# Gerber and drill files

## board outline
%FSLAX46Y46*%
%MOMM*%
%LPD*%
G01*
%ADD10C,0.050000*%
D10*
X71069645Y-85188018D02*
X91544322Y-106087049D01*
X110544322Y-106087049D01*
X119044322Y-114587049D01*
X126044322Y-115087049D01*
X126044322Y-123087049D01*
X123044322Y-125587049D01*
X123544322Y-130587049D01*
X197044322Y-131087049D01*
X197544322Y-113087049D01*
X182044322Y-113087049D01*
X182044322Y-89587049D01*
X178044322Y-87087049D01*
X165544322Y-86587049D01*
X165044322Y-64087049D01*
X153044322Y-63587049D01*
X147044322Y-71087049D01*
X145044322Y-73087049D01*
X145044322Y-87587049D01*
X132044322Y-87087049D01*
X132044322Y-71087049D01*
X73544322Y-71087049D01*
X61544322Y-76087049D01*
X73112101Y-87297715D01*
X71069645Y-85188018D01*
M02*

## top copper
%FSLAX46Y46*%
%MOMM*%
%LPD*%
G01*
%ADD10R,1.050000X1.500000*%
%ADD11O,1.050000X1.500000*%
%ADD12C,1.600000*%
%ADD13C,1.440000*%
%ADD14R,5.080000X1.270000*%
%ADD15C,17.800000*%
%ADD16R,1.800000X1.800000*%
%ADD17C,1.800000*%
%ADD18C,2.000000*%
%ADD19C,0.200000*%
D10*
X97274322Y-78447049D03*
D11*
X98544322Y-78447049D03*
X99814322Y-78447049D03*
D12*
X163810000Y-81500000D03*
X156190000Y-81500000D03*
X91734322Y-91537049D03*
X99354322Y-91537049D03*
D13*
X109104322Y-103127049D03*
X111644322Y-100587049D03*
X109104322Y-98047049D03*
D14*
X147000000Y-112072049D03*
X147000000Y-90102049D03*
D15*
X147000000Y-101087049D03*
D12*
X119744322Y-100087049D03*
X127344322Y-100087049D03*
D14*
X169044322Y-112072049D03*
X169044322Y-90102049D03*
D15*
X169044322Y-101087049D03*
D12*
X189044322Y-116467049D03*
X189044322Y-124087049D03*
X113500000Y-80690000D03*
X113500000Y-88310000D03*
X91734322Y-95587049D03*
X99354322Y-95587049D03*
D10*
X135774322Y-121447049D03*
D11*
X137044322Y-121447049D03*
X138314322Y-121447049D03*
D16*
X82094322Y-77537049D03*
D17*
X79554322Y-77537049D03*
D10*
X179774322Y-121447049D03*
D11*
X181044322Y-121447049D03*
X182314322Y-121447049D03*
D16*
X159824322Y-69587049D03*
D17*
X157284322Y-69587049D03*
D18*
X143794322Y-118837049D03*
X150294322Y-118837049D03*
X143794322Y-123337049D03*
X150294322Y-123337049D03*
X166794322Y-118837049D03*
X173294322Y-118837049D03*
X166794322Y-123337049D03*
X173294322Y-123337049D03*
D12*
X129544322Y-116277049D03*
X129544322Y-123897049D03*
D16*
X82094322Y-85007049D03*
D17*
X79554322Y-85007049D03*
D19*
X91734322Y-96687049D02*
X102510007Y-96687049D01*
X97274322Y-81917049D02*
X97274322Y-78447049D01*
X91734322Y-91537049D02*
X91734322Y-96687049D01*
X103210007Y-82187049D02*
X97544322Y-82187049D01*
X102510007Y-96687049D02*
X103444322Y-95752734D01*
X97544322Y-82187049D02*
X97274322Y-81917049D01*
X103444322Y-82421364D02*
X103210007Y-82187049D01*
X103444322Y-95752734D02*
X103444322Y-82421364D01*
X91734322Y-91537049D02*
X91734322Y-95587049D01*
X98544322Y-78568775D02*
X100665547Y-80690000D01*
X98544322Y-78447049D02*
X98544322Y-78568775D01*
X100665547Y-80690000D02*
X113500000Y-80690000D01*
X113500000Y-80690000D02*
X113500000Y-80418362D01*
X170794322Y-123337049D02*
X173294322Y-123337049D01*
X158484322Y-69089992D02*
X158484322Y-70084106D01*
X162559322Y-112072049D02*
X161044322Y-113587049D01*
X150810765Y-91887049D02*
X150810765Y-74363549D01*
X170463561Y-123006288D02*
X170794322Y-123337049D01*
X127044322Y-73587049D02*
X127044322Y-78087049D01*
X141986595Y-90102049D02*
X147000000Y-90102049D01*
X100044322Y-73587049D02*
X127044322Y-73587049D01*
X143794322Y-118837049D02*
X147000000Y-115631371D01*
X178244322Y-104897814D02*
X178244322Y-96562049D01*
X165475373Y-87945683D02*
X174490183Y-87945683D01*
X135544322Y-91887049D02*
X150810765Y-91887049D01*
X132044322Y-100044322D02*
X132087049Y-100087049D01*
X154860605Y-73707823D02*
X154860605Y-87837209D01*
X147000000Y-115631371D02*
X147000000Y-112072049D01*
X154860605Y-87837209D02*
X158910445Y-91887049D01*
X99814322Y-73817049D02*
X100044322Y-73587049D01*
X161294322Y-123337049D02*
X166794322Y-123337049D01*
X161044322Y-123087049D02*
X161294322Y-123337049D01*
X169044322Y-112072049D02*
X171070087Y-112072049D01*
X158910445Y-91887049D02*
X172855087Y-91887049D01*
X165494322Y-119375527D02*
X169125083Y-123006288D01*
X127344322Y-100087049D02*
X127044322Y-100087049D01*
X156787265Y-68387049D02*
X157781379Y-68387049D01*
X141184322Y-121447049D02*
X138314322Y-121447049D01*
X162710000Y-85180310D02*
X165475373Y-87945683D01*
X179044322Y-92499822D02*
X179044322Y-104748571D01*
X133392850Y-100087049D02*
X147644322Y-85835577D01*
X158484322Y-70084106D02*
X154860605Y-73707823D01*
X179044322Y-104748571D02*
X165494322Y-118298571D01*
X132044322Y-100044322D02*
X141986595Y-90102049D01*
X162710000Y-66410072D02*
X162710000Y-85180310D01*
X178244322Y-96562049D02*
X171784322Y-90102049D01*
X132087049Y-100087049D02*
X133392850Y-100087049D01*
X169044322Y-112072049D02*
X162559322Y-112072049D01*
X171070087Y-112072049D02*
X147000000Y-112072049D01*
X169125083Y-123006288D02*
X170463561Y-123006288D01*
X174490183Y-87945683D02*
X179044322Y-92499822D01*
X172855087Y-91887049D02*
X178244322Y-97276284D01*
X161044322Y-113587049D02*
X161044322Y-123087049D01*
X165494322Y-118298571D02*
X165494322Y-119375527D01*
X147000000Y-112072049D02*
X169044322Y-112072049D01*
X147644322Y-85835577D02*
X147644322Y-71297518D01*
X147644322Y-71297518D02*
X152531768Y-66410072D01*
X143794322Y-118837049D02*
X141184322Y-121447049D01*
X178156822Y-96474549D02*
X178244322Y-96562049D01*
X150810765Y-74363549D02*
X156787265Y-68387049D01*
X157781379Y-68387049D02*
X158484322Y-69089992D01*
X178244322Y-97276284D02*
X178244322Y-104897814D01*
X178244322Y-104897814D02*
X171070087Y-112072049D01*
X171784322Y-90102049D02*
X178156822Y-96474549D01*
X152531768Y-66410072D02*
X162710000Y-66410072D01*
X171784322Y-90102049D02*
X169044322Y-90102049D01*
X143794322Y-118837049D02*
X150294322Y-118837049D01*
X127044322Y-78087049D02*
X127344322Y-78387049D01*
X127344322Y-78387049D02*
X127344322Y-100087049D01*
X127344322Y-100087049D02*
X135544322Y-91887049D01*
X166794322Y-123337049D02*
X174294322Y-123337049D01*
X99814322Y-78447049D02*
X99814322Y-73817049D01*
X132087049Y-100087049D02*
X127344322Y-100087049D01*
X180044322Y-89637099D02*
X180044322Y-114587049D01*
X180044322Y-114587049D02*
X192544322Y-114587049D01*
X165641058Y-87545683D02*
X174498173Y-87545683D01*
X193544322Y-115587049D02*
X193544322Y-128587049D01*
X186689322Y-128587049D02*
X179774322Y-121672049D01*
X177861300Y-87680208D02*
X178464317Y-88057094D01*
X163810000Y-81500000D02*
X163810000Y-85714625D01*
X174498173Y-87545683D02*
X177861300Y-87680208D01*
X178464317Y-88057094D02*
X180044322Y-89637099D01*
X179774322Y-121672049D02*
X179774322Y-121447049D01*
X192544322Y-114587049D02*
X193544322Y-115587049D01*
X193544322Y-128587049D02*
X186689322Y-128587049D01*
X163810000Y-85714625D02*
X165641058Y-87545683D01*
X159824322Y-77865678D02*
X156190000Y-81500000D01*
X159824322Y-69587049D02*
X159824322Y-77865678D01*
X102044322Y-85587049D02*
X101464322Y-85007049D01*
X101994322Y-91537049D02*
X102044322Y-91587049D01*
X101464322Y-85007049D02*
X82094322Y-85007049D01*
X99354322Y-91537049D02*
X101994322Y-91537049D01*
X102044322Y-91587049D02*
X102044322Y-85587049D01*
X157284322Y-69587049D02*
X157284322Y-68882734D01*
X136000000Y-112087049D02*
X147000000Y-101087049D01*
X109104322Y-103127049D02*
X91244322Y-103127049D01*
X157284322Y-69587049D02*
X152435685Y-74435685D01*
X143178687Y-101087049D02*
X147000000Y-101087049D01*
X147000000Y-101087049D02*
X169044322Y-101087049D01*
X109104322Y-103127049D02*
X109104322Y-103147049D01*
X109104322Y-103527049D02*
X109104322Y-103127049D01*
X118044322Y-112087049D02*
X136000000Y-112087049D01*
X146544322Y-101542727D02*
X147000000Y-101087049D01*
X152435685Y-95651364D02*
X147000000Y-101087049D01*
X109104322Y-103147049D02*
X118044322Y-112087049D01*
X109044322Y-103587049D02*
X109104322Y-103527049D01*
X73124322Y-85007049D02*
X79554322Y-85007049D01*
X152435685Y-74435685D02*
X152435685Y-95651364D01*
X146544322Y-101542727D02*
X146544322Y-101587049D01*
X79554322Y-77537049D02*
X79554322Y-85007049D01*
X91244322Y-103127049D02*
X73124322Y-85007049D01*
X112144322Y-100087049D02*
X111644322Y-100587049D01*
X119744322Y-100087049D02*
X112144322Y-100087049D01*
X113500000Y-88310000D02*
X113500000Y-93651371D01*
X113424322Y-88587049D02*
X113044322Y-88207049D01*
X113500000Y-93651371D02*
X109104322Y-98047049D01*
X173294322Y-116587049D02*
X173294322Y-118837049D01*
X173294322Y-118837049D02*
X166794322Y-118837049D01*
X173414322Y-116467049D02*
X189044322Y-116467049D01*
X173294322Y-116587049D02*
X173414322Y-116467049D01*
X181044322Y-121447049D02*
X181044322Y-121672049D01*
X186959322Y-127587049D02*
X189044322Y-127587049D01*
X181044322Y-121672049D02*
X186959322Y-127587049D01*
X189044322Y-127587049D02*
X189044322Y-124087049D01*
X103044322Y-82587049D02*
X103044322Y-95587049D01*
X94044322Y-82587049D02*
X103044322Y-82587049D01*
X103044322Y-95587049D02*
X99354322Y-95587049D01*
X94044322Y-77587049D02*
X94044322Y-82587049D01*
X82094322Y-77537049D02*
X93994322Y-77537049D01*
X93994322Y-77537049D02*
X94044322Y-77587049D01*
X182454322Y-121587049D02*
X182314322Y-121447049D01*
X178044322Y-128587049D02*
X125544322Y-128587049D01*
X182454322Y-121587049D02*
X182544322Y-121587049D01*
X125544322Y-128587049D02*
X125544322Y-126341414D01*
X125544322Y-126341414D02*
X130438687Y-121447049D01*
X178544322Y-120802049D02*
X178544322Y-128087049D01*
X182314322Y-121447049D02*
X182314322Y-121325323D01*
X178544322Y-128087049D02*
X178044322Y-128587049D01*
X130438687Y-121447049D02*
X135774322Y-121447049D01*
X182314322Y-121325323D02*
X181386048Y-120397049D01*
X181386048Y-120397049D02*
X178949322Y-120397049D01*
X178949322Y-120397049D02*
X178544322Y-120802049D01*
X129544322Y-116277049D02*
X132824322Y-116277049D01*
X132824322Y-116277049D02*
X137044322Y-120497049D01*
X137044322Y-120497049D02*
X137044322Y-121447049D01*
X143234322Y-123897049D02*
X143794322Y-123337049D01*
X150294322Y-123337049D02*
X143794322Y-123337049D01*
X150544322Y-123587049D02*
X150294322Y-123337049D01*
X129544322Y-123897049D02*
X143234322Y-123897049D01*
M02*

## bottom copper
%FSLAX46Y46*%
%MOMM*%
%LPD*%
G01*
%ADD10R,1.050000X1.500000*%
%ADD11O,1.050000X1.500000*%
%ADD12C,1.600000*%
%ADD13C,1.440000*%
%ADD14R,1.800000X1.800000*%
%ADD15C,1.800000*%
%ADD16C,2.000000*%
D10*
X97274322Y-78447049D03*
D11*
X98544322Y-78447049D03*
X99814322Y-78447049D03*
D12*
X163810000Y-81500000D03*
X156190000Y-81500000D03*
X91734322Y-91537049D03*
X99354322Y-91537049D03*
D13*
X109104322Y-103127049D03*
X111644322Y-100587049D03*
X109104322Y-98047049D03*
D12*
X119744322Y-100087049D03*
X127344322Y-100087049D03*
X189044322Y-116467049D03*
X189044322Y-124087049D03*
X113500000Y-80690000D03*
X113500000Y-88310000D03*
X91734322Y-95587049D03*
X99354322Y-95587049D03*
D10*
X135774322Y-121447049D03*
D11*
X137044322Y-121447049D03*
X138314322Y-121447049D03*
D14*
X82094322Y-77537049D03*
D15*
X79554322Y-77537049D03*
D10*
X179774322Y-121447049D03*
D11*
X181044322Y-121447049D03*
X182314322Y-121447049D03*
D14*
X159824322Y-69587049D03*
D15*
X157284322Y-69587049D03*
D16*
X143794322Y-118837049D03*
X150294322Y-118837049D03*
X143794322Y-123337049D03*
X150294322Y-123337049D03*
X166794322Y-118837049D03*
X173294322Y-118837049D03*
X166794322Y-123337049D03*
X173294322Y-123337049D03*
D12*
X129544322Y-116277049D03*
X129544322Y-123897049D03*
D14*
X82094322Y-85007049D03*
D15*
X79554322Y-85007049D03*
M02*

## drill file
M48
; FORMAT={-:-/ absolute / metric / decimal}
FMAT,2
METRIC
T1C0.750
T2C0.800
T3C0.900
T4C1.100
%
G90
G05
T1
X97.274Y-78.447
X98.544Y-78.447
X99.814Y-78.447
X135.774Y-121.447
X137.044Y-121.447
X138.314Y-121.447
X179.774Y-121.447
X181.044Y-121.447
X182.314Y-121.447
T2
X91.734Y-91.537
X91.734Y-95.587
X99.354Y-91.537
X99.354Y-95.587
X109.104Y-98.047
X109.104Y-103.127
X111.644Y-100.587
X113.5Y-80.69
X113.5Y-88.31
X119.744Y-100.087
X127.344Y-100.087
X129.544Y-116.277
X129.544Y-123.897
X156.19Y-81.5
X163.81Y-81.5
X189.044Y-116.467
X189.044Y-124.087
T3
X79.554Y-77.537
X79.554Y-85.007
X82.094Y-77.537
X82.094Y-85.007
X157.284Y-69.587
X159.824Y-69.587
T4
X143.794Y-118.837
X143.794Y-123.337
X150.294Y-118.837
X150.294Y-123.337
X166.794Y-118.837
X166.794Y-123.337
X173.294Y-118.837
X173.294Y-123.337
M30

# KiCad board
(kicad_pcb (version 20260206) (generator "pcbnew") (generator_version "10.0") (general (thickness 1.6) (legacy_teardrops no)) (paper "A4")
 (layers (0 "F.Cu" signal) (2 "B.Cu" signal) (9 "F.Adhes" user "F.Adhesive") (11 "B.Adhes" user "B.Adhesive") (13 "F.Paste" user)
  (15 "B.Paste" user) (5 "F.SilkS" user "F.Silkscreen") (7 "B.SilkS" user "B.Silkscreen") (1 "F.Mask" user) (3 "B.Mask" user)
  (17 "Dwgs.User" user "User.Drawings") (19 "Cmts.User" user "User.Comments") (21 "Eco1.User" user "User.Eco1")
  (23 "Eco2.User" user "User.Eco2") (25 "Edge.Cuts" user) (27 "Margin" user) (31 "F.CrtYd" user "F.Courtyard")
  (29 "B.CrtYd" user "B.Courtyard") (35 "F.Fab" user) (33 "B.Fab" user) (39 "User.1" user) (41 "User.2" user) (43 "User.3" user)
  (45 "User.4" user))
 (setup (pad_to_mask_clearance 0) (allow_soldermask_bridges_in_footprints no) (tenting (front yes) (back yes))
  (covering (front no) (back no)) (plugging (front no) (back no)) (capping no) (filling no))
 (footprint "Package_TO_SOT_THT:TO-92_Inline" (layer "F.Cu") (at 97.274322 78.447049)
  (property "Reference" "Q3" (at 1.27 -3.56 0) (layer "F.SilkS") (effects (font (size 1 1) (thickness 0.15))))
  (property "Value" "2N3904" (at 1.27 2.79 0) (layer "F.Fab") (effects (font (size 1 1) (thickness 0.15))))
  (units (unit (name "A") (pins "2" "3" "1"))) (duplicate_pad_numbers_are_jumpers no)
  (pad "1" thru_hole rect (at 0 0) (size 1.05 1.5) (drill 0.75) (layers "*.Cu" "*.Mask") (remove_unused_layers no) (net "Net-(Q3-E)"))
  (pad "2" thru_hole oval (at 1.27 0) (size 1.05 1.5) (drill 0.75) (layers "*.Cu" "*.Mask") (remove_unused_layers no) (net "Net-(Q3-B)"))
  (pad "3" thru_hole oval (at 2.54 0) (size 1.05 1.5) (drill 0.75) (layers "*.Cu" "*.Mask") (remove_unused_layers no) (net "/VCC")))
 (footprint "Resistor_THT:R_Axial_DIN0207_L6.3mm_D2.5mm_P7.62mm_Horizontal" (layer "F.Cu") (at 163.81 81.5 180)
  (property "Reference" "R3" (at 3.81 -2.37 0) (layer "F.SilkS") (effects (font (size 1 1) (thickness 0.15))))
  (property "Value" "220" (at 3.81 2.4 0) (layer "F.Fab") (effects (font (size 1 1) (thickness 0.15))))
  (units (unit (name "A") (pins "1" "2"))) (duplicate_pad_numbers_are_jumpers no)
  (pad "1" thru_hole circle (at 0 0 180) (size 1.6 1.6) (drill 0.8) (layers "*.Cu" "*.Mask") (remove_unused_layers no) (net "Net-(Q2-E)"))
  (pad "2" thru_hole circle (at 7.62 0 180) (size 1.6 1.6) (drill 0.8) (layers "*.Cu" "*.Mask") (remove_unused_layers no) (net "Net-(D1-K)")))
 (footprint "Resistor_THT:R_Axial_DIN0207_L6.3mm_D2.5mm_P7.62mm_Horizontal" (layer "F.Cu") (at 91.734322 91.537049)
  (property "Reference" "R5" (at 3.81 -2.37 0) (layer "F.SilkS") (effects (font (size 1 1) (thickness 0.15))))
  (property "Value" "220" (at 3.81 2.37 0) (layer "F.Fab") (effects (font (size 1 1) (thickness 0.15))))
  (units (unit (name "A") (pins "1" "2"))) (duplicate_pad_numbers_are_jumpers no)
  (pad "1" thru_hole circle (at 0 0) (size 1.6 1.6) (drill 0.8) (layers "*.Cu" "*.Mask") (remove_unused_layers no) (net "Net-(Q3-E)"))
  (pad "2" thru_hole circle (at 7.62 0) (size 1.6 1.6) (drill 0.8) (layers "*.Cu" "*.Mask") (remove_unused_layers no) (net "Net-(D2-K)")))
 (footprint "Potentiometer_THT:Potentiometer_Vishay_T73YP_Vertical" (layer "F.Cu") (at 109.104322 103.127049)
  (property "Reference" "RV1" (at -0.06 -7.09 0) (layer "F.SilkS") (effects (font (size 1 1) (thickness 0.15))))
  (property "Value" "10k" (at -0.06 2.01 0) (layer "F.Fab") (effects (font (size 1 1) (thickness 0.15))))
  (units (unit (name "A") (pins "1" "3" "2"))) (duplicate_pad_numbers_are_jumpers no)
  (pad "1" thru_hole circle (at 0 0) (size 1.44 1.44) (drill 0.8) (layers "*.Cu" "*.Mask") (remove_unused_layers no) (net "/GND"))
  (pad "2" thru_hole circle (at 2.54 -2.54) (size 1.44 1.44) (drill 0.8) (layers "*.Cu" "*.Mask") (remove_unused_layers no)
   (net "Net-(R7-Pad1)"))
  (pad "3" thru_hole circle (at 0 -5.08) (size 1.44 1.44) (drill 0.8) (layers "*.Cu" "*.Mask") (remove_unused_layers no)
   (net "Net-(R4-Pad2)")))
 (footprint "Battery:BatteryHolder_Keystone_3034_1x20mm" (layer "F.Cu") (at 147 101.087049 90)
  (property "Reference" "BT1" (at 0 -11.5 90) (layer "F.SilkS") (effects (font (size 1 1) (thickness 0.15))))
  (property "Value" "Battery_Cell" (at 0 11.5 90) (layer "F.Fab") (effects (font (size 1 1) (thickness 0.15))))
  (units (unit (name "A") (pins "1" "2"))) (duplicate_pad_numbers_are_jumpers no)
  (pad "1" smd rect (at -10.985 0 90) (size 1.27 5.08) (layers "F.Cu" "F.Mask" "F.Paste") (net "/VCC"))
  (pad "1" smd rect (at 10.985 0 90) (size 1.27 5.08) (layers "F.Cu" "F.Mask" "F.Paste") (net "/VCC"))
  (pad "2" smd circle (at 0 0 90) (size 17.8 17.8) (layers "F.Cu" "F.Mask") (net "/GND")))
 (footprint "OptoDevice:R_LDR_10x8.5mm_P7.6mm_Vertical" (layer "F.Cu") (at 119.744322 100.087049)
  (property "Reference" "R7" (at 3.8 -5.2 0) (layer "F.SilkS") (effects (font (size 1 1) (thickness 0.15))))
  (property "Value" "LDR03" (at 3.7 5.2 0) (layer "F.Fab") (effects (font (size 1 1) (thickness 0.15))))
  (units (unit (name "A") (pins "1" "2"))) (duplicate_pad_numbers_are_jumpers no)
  (pad "1" thru_hole circle (at 0 0) (size 1.6 1.6) (drill 0.8) (layers "*.Cu" "*.Mask") (remove_unused_layers no) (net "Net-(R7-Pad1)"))
  (pad "2" thru_hole circle (at 7.6 0) (size 1.6 1.6) (drill 0.8) (layers "*.Cu" "*.Mask") (remove_unused_layers no) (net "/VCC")))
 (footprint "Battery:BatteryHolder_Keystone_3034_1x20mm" (layer "F.Cu") (at 169.044322 101.087049 90)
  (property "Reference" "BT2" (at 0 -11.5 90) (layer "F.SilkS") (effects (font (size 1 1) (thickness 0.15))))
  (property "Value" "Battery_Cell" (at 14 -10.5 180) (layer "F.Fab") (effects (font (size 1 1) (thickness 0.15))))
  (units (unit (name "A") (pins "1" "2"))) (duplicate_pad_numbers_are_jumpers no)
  (pad "1" smd rect (at -10.985 0 90) (size 1.27 5.08) (layers "F.Cu" "F.Mask" "F.Paste") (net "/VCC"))
  (pad "1" smd rect (at 10.985 0 90) (size 1.27 5.08) (layers "F.Cu" "F.Mask" "F.Paste") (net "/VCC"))
  (pad "2" smd circle (at 0 0 90) (size 17.8 17.8) (layers "F.Cu" "F.Mask") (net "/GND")))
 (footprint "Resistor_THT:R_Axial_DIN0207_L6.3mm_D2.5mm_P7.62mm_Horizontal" (layer "F.Cu") (at 189.044322 116.467049 -90)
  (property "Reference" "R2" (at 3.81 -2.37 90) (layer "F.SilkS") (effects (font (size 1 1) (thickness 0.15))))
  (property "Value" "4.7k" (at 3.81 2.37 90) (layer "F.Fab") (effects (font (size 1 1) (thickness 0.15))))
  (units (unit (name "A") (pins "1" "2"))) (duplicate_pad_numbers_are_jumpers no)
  (pad "1" thru_hole circle (at 0 0 270) (size 1.6 1.6) (drill 0.8) (layers "*.Cu" "*.Mask") (remove_unused_layers no) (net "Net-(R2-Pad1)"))
  (pad "2" thru_hole circle (at 7.62 0 270) (size 1.6 1.6) (drill 0.8) (layers "*.Cu" "*.Mask") (remove_unused_layers no) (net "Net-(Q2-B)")))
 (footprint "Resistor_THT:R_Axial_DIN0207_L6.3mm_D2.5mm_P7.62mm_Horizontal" (layer "F.Cu") (at 113.5 80.69 -90)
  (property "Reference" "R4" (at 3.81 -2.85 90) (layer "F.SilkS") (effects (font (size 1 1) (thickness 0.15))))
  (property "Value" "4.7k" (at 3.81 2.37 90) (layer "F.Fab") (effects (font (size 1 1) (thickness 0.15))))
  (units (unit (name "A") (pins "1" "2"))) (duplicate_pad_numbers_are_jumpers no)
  (pad "1" thru_hole circle (at 0 0 270) (size 1.6 1.6) (drill 0.8) (layers "*.Cu" "*.Mask") (remove_unused_layers no) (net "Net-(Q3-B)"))
  (pad "2" thru_hole circle (at 7.62 0 270) (size 1.6 1.6) (drill 0.8) (layers "*.Cu" "*.Mask") (remove_unused_layers no)
   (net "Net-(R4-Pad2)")))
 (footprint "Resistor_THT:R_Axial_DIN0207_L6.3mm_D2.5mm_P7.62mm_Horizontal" (layer "F.Cu") (at 91.734322 95.587049)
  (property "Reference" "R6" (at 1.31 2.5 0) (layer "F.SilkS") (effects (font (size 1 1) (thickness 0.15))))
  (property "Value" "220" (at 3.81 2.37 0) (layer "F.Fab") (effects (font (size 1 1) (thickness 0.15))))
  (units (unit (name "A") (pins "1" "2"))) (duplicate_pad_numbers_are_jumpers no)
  (pad "1" thru_hole circle (at 0 0) (size 1.6 1.6) (drill 0.8) (layers "*.Cu" "*.Mask") (remove_unused_layers no) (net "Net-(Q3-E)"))
  (pad "2" thru_hole circle (at 7.62 0) (size 1.6 1.6) (drill 0.8) (layers "*.Cu" "*.Mask") (remove_unused_layers no) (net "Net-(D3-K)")))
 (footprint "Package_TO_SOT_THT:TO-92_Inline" (layer "F.Cu") (at 135.774322 121.447049)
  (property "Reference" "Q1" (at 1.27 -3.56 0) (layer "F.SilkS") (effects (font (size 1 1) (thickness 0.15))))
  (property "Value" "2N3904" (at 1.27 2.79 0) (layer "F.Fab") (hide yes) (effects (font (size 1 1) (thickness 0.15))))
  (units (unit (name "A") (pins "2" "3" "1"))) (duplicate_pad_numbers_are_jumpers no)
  (pad "1" thru_hole rect (at 0 0) (size 1.05 1.5) (drill 0.75) (layers "*.Cu" "*.Mask") (remove_unused_layers no) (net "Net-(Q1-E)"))
  (pad "2" thru_hole oval (at 1.27 0) (size 1.05 1.5) (drill 0.75) (layers "*.Cu" "*.Mask") (remove_unused_layers no) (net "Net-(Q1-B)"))
  (pad "3" thru_hole oval (at 2.54 0) (size 1.05 1.5) (drill 0.75) (layers "*.Cu" "*.Mask") (remove_unused_layers no) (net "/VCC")))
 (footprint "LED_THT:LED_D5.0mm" (layer "F.Cu") (at 82.094322 77.537049 180)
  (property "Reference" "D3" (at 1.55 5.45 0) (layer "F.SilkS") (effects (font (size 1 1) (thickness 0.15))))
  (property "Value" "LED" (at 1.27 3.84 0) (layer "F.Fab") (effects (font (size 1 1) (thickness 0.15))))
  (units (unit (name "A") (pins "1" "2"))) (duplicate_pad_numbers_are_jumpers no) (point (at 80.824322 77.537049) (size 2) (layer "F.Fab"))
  (pad "1" thru_hole rect (at 0 0 180) (size 1.8 1.8) (drill 0.9) (layers "*.Cu" "*.Mask") (remove_unused_layers no) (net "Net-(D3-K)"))
  (pad "2" thru_hole circle (at 2.54 0 180) (size 1.8 1.8) (drill 0.9) (layers "*.Cu" "*.Mask") (remove_unused_layers no) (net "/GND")))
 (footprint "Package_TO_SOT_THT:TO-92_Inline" (layer "F.Cu") (at 179.774322 121.447049)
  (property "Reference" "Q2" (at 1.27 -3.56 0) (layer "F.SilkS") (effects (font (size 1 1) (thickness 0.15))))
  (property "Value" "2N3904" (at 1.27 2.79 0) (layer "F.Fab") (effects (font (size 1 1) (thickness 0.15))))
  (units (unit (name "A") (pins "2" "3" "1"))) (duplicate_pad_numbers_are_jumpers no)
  (pad "1" thru_hole rect (at 0 0) (size 1.05 1.5) (drill 0.75) (layers "*.Cu" "*.Mask") (remove_unused_layers no) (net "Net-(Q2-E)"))
  (pad "2" thru_hole oval (at 1.27 0) (size 1.05 1.5) (drill 0.75) (layers "*.Cu" "*.Mask") (remove_unused_layers no) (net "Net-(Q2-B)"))
  (pad "3" thru_hole oval (at 2.54 0) (size 1.05 1.5) (drill 0.75) (layers "*.Cu" "*.Mask") (remove_unused_layers no) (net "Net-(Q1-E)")))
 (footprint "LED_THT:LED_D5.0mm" (layer "F.Cu") (at 159.824322 69.587049 180)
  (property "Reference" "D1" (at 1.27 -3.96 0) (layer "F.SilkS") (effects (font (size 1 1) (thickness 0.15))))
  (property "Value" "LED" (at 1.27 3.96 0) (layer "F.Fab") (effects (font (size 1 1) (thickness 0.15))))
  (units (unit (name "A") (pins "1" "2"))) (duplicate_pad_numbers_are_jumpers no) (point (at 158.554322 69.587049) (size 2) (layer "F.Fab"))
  (pad "1" thru_hole rect (at 0 0 180) (size 1.8 1.8) (drill 0.9) (layers "*.Cu" "*.Mask") (remove_unused_layers no) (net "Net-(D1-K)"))
  (pad "2" thru_hole circle (at 2.54 0 180) (size 1.8 1.8) (drill 0.9) (layers "*.Cu" "*.Mask") (remove_unused_layers no) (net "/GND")))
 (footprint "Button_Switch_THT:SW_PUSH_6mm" (layer "F.Cu") (at 143.794322 118.837049)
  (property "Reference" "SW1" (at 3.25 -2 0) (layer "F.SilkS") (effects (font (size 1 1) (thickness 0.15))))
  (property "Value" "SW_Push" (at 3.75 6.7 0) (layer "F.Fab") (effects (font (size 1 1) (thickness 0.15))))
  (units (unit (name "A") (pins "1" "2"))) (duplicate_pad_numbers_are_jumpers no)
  (pad "1" thru_hole circle (at 0 0 90) (size 2 2) (drill 1.1) (layers "*.Cu" "*.Mask") (remove_unused_layers no) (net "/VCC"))
  (pad "1" thru_hole circle (at 6.5 0 90) (size 2 2) (drill 1.1) (layers "*.Cu" "*.Mask") (remove_unused_layers no) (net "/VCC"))
  (pad "2" thru_hole circle (at 0 4.5 90) (size 2 2) (drill 1.1) (layers "*.Cu" "*.Mask") (remove_unused_layers no) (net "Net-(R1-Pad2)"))
  (pad "2" thru_hole circle (at 6.5 4.5 90) (size 2 2) (drill 1.1) (layers "*.Cu" "*.Mask") (remove_unused_layers no) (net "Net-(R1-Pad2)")))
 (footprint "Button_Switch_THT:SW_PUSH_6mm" (layer "F.Cu") (at 166.794322 118.837049)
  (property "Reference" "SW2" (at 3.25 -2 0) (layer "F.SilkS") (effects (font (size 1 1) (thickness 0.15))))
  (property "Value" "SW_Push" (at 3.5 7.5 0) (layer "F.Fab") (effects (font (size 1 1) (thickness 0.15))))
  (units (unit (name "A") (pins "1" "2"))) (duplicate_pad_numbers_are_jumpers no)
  (pad "1" thru_hole circle (at 0 0 90) (size 2 2) (drill 1.1) (layers "*.Cu" "*.Mask") (remove_unused_layers no) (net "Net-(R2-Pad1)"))
  (pad "1" thru_hole circle (at 6.5 0 90) (size 2 2) (drill 1.1) (layers "*.Cu" "*.Mask") (remove_unused_layers no) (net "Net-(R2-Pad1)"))
  (pad "2" thru_hole circle (at 0 4.5 90) (size 2 2) (drill 1.1) (layers "*.Cu" "*.Mask") (remove_unused_layers no) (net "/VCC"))
  (pad "2" thru_hole circle (at 6.5 4.5 90) (size 2 2) (drill 1.1) (layers "*.Cu" "*.Mask") (remove_unused_layers no) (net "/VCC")))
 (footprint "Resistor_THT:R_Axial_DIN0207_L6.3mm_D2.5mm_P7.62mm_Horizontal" (layer "F.Cu") (at 129.544322 116.277049 -90)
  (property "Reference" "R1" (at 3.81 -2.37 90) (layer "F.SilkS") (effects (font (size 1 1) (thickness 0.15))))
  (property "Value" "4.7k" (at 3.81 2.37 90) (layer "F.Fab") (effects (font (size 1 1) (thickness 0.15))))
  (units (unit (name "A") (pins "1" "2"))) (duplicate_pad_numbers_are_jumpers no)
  (pad "1" thru_hole circle (at 0 0 270) (size 1.6 1.6) (drill 0.8) (layers "*.Cu" "*.Mask") (remove_unused_layers no) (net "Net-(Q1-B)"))
  (pad "2" thru_hole circle (at 7.62 0 270) (size 1.6 1.6) (drill 0.8) (layers "*.Cu" "*.Mask") (remove_unused_layers no)
   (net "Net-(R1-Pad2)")))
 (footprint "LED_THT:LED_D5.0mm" (layer "F.Cu") (at 82.094322 85.007049 180)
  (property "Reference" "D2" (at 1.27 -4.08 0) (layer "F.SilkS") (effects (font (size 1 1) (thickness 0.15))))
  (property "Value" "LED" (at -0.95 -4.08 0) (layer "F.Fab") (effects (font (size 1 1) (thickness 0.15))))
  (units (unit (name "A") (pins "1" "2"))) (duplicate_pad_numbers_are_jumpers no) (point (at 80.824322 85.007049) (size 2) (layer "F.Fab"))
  (pad "1" thru_hole rect (at 0 0 180) (size 1.8 1.8) (drill 0.9) (layers "*.Cu" "*.Mask") (remove_unused_layers no) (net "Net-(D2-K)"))
  (pad "2" thru_hole circle (at 2.54 0 180) (size 1.8 1.8) (drill 0.9) (layers "*.Cu" "*.Mask") (remove_unused_layers no) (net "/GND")))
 (gr_poly
  (pts (xy 71.069645 85.188018) (xy 91.544322 106.087049) (xy 110.544322 106.087049) (xy 119.044322 114.587049) (xy 126.044322 115.087049)
   (xy 126.044322 123.087049) (xy 123.044322 125.587049) (xy 123.544322 130.587049) (xy 197.044322 131.087049) (xy 197.544322 113.087049)
   (xy 182.044322 113.087049) (xy 182.044322 89.587049) (xy 178.044322 87.087049) (xy 165.544322 86.587049) (xy 165.044322 64.087049)
   (xy 153.044322 63.587049) (xy 147.044322 71.087049) (xy 145.044322 73.087049) (xy 145.044322 87.587049) (xy 132.044322 87.087049)
   (xy 132.044322 71.087049) (xy 73.544322 71.087049) (xy 61.544322 76.087049) (xy 73.112101 87.297715))
  (stroke (width 0.05) (type solid)) (fill no) (layer "Edge.Cuts"))
 (segment (start 91.734322 96.687049) (end 102.510007 96.687049) (width 0.2) (layer "F.Cu") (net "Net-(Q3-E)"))
 (segment (start 97.274322 81.917049) (end 97.274322 78.447049) (width 0.2) (layer "F.Cu") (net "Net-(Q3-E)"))
 (segment (start 91.734322 91.537049) (end 91.734322 96.687049) (width 0.2) (layer "F.Cu") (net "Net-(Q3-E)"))
 (segment (start 103.210007 82.187049) (end 97.544322 82.187049) (width 0.2) (layer "F.Cu") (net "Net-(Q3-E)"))
 (segment (start 102.510007 96.687049) (end 103.444322 95.752734) (width 0.2) (layer "F.Cu") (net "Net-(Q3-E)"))
 (segment (start 97.544322 82.187049) (end 97.274322 81.917049) (width 0.2) (layer "F.Cu") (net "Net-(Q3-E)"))
 (segment (start 103.444322 82.421364) (end 103.210007 82.187049) (width 0.2) (layer "F.Cu") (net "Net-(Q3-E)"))
 (segment (start 103.444322 95.752734) (end 103.444322 82.421364) (width 0.2) (layer "F.Cu") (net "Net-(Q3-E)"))
 (segment (start 91.734322 91.537049) (end 91.734322 95.587049) (width 0.2) (layer "F.Cu") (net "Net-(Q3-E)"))
 (segment (start 98.544322 78.568775) (end 100.665547 80.69) (width 0.2) (layer "F.Cu") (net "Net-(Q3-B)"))
 (segment (start 98.544322 78.447049) (end 98.544322 78.568775) (width 0.2) (layer "F.Cu") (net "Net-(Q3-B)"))
 (segment (start 100.665547 80.69) (end 113.5 80.69) (width 0.2) (layer "F.Cu") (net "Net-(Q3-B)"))
 (segment (start 113.5 80.69) (end 113.5 80.418362) (width 0.2) (layer "F.Cu") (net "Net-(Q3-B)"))
 (segment (start 170.794322 123.337049) (end 173.294322 123.337049) (width 0.2) (layer "F.Cu") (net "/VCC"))
 (segment (start 158.484322 69.089992) (end 158.484322 70.084106) (width 0.2) (layer "F.Cu") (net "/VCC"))
 (segment (start 162.559322 112.072049) (end 161.044322 113.587049) (width 0.2) (layer "F.Cu") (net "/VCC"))
 (segment (start 150.810765 91.887049) (end 150.810765 74.363549) (width 0.2) (layer "F.Cu") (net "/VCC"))
 (segment (start 170.463561 123.006288) (end 170.794322 123.337049) (width 0.2) (layer "F.Cu") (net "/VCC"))
 (segment (start 127.044322 73.587049) (end 127.044322 78.087049) (width 0.2) (layer "F.Cu") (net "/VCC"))
 (segment (start 141.986595 90.102049) (end 147 90.102049) (width 0.2) (layer "F.Cu") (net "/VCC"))
 (segment (start 100.044322 73.587049) (end 127.044322 73.587049) (width 0.2) (layer "F.Cu") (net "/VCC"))
 (segment (start 143.794322 118.837049) (end 147 115.631371) (width 0.2) (layer "F.Cu") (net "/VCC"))
 (segment (start 178.244322 104.897814) (end 178.244322 96.562049) (width 0.2) (layer "F.Cu") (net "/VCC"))
 (segment (start 165.475373 87.945683) (end 174.490183 87.945683) (width 0.2) (layer "F.Cu") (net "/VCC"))
 (segment (start 135.544322 91.887049) (end 150.810765 91.887049) (width 0.2) (layer "F.Cu") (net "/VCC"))
 (segment (start 132.044322 100.044322) (end 132.087049 100.087049) (width 0.2) (layer "F.Cu") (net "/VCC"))
 (segment (start 154.860605 73.707823) (end 154.860605 87.837209) (width 0.2) (layer "F.Cu") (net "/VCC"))
 (segment (start 147 115.631371) (end 147 112.072049) (width 0.2) (layer "F.Cu") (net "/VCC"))
 (segment (start 154.860605 87.837209) (end 158.910445 91.887049) (width 0.2) (layer "F.Cu") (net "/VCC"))
 (segment (start 99.814322 73.817049) (end 100.044322 73.587049) (width 0.2) (layer "F.Cu") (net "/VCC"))
 (segment (start 161.294322 123.337049) (end 166.794322 123.337049) (width 0.2) (layer "F.Cu") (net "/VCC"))
 (segment (start 161.044322 123.087049) (end 161.294322 123.337049) (width 0.2) (layer "F.Cu") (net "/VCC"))
 (segment (start 169.044322 112.072049) (end 171.070087 112.072049) (width 0.2) (layer "F.Cu") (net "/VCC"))
 (segment (start 158.910445 91.887049) (end 172.855087 91.887049) (width 0.2) (layer "F.Cu") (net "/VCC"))
 (segment (start 165.494322 119.375527) (end 169.125083 123.006288) (width 0.2) (layer "F.Cu") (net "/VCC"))
 (segment (start 127.344322 100.087049) (end 127.044322 100.087049) (width 0.2) (layer "F.Cu") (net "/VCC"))
 (segment (start 156.787265 68.387049) (end 157.781379 68.387049) (width 0.2) (layer "F.Cu") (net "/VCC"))
 (segment (start 141.184322 121.447049) (end 138.314322 121.447049) (width 0.2) (layer "F.Cu") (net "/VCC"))
 (segment (start 162.71 85.18031) (end 165.475373 87.945683) (width 0.2) (layer "F.Cu") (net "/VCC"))
 (segment (start 179.044322 92.499822) (end 179.044322 104.748571) (width 0.2) (layer "F.Cu") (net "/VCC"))
 (segment (start 133.39285 100.087049) (end 147.644322 85.835577) (width 0.2) (layer "F.Cu") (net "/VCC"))
 (segment (start 158.484322 70.084106) (end 154.860605 73.707823) (width 0.2) (layer "F.Cu") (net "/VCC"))
 (segment (start 179.044322 104.748571) (end 165.494322 118.298571) (width 0.2) (layer "F.Cu") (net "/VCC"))
 (segment (start 132.044322 100.044322) (end 141.986595 90.102049) (width 0.2) (layer "F.Cu") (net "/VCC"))
 (segment (start 162.71 66.410072) (end 162.71 85.18031) (width 0.2) (layer "F.Cu") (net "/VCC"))
 (segment (start 178.244322 96.562049) (end 171.784322 90.102049) (width 0.2) (layer "F.Cu") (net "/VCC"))
 (segment (start 132.087049 100.087049) (end 133.39285 100.087049) (width 0.2) (layer "F.Cu") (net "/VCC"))
 (segment (start 169.044322 112.072049) (end 162.559322 112.072049) (width 0.2) (layer "F.Cu") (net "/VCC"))
 (segment (start 171.070087 112.072049) (end 147 112.072049) (width 0.2) (layer "F.Cu") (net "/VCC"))
 (segment (start 169.125083 123.006288) (end 170.463561 123.006288) (width 0.2) (layer "F.Cu") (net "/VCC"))
 (segment (start 174.490183 87.945683) (end 179.044322 92.499822) (width 0.2) (layer "F.Cu") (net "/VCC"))
 (segment (start 172.855087 91.887049) (end 178.244322 97.276284) (width 0.2) (layer "F.Cu") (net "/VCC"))
 (segment (start 161.044322 113.587049) (end 161.044322 123.087049) (width 0.2) (layer "F.Cu") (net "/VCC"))
 (segment (start 165.494322 118.298571) (end 165.494322 119.375527) (width 0.2) (layer "F.Cu") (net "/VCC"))
 (segment (start 147 112.072049) (end 169.044322 112.072049) (width 0.2) (layer "F.Cu") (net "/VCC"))
 (segment (start 147.644322 85.835577) (end 147.644322 71.297518) (width 0.2) (layer "F.Cu") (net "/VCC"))
 (segment (start 147.644322 71.297518) (end 152.531768 66.410072) (width 0.2) (layer "F.Cu") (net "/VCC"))
 (segment (start 143.794322 118.837049) (end 141.184322 121.447049) (width 0.2) (layer "F.Cu") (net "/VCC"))
 (segment (start 178.156822 96.474549) (end 178.244322 96.562049) (width 0.2) (layer "F.Cu") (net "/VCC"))
 (segment (start 150.810765 74.363549) (end 156.787265 68.387049) (width 0.2) (layer "F.Cu") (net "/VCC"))
 (segment (start 157.781379 68.387049) (end 158.484322 69.089992) (width 0.2) (layer "F.Cu") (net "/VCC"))
 (segment (start 178.244322 97.276284) (end 178.244322 104.897814) (width 0.2) (layer "F.Cu") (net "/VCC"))
 (segment (start 178.244322 104.897814) (end 171.070087 112.072049) (width 0.2) (layer "F.Cu") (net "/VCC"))
 (segment (start 171.784322 90.102049) (end 178.156822 96.474549) (width 0.2) (layer "F.Cu") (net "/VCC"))
 (segment (start 152.531768 66.410072) (end 162.71 66.410072) (width 0.2) (layer "F.Cu") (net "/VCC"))
 (segment (start 171.784322 90.102049) (end 169.044322 90.102049) (width 0.2) (layer "F.Cu") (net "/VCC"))
 (segment (start 143.794322 118.837049) (end 150.294322 118.837049) (width 0.2) (layer "F.Cu") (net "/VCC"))
 (segment (start 127.044322 78.087049) (end 127.344322 78.387049) (width 0.2) (layer "F.Cu") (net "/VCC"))
 (segment (start 127.344322 78.387049) (end 127.344322 100.087049) (width 0.2) (layer "F.Cu") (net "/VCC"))
 (segment (start 127.344322 100.087049) (end 135.544322 91.887049) (width 0.2) (layer "F.Cu") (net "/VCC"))
 (segment (start 166.794322 123.337049) (end 174.294322 123.337049) (width 0.2) (layer "F.Cu") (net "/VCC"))
 (segment (start 99.814322 78.447049) (end 99.814322 73.817049) (width 0.2) (layer "F.Cu") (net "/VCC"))
 (segment (start 132.087049 100.087049) (end 127.344322 100.087049) (width 0.2) (layer "F.Cu") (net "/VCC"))
 (segment (start 180.044322 89.637099) (end 180.044322 114.587049) (width 0.2) (layer "F.Cu") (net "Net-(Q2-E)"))
 (segment (start 180.044322 114.587049) (end 192.544322 114.587049) (width 0.2) (layer "F.Cu") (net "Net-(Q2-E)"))
 (segment (start 165.641058 87.545683) (end 174.498173 87.545683) (width 0.2) (layer "F.Cu") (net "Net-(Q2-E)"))
 (segment (start 193.544322 115.587049) (end 193.544322 128.587049) (width 0.2) (layer "F.Cu") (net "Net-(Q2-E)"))
 (segment (start 186.689322 128.587049) (end 179.774322 121.672049) (width 0.2) (layer "F.Cu") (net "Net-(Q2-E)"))
 (segment (start 177.8613 87.680208) (end 178.464317 88.057094) (width 0.2) (layer "F.Cu") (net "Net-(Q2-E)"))
 (segment (start 163.81 81.5) (end 163.81 85.714625) (width 0.2) (layer "F.Cu") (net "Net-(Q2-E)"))
 (segment (start 174.498173 87.545683) (end 177.8613 87.680208) (width 0.2) (layer "F.Cu") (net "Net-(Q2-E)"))
 (segment (start 178.464317 88.057094) (end 180.044322 89.637099) (width 0.2) (layer "F.Cu") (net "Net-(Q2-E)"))
 (segment (start 179.774322 121.672049) (end 179.774322 121.447049) (width 0.2) (layer "F.Cu") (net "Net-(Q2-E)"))
 (segment (start 192.544322 114.587049) (end 193.544322 115.587049) (width 0.2) (layer "F.Cu") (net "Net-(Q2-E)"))
 (segment (start 193.544322 128.587049) (end 186.689322 128.587049) (width 0.2) (layer "F.Cu") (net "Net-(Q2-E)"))
 (segment (start 163.81 85.714625) (end 165.641058 87.545683) (width 0.2) (layer "F.Cu") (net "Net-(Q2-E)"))
 (segment (start 159.824322 77.865678) (end 156.19 81.5) (width 0.2) (layer "F.Cu") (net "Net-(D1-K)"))
 (segment (start 159.824322 69.587049) (end 159.824322 77.865678) (width 0.2) (layer "F.Cu") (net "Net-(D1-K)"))
 (segment (start 102.044322 85.587049) (end 101.464322 85.007049) (width 0.2) (layer "F.Cu") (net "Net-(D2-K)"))
 (segment (start 101.994322 91.537049) (end 102.044322 91.587049) (width 0.2) (layer "F.Cu") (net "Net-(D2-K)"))
 (segment (start 101.464322 85.007049) (end 82.094322 85.007049) (width 0.2) (layer "F.Cu") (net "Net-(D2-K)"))
 (segment (start 99.354322 91.537049) (end 101.994322 91.537049) (width 0.2) (layer "F.Cu") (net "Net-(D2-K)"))
 (segment (start 102.044322 91.587049) (end 102.044322 85.587049) (width 0.2) (layer "F.Cu") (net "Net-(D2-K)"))
 (segment (start 157.284322 69.587049) (end 157.284322 68.882734) (width 0.2) (layer "F.Cu") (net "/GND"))
 (segment (start 136 112.087049) (end 147 101.087049) (width 0.2) (layer "F.Cu") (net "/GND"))
 (segment (start 109.104322 103.127049) (end 91.244322 103.127049) (width 0.2) (layer "F.Cu") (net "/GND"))
 (segment (start 157.284322 69.587049) (end 152.435685 74.435685) (width 0.2) (layer "F.Cu") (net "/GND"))
 (segment (start 143.178687 101.087049) (end 147 101.087049) (width 0.2) (layer "F.Cu") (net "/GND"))
 (segment (start 147 101.087049) (end 169.044322 101.087049) (width 0.2) (layer "F.Cu") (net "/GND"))
 (segment (start 109.104322 103.127049) (end 109.104322 103.147049) (width 0.2) (layer "F.Cu") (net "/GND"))
 (segment (start 109.104322 103.527049) (end 109.104322 103.127049) (width 0.2) (layer "F.Cu") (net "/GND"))
 (segment (start 118.044322 112.087049) (end 136 112.087049) (width 0.2) (layer "F.Cu") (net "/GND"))
 (segment (start 146.544322 101.542727) (end 147 101.087049) (width 0.2) (layer "F.Cu") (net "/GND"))
 (segment (start 152.435685 95.651364) (end 147 101.087049) (width 0.2) (layer "F.Cu") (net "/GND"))
 (segment (start 109.104322 103.147049) (end 118.044322 112.087049) (width 0.2) (layer "F.Cu") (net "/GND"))
 (segment (start 109.044322 103.587049) (end 109.104322 103.527049) (width 0.2) (layer "F.Cu") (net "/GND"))
 (segment (start 73.124322 85.007049) (end 79.554322 85.007049) (width 0.2) (layer "F.Cu") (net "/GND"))
 (segment (start 152.435685 74.435685) (end 152.435685 95.651364) (width 0.2) (layer "F.Cu") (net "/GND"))
 (segment (start 146.544322 101.542727) (end 146.544322 101.587049) (width 0.2) (layer "F.Cu") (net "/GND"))
 (segment (start 79.554322 77.537049) (end 79.554322 85.007049) (width 0.2) (layer "F.Cu") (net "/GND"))
 (segment (start 91.244322 103.127049) (end 73.124322 85.007049) (width 0.2) (layer "F.Cu") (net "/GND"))
 (segment (start 112.144322 100.087049) (end 111.644322 100.587049) (width 0.2) (layer "F.Cu") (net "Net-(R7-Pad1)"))
 (segment (start 119.744322 100.087049) (end 112.144322 100.087049) (width 0.2) (layer "F.Cu") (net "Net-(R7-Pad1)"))
 (segment (start 113.5 88.31) (end 113.5 93.651371) (width 0.2) (layer "F.Cu") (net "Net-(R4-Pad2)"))
 (segment (start 113.424322 88.587049) (end 113.044322 88.207049) (width 0.2) (layer "F.Cu") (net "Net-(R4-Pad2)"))
 (segment (start 113.5 93.651371) (end 109.104322 98.047049) (width 0.2) (layer "F.Cu") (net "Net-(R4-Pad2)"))
 (segment (start 173.294322 116.587049) (end 173.294322 118.837049) (width 0.2) (layer "F.Cu") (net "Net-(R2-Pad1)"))
 (segment (start 173.294322 118.837049) (end 166.794322 118.837049) (width 0.2) (layer "F.Cu") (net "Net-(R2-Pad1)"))
 (segment (start 173.414322 116.467049) (end 189.044322 116.467049) (width 0.2) (layer "F.Cu") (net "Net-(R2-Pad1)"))
 (segment (start 173.294322 116.587049) (end 173.414322 116.467049) (width 0.2) (layer "F.Cu") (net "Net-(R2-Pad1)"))
 (segment (start 181.044322 121.447049) (end 181.044322 121.672049) (width 0.2) (layer "F.Cu") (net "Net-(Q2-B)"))
 (segment (start 186.959322 127.587049) (end 189.044322 127.587049) (width 0.2) (layer "F.Cu") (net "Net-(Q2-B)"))
 (segment (start 181.044322 121.672049) (end 186.959322 127.587049) (width 0.2) (layer "F.Cu") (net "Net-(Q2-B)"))
 (segment (start 189.044322 127.587049) (end 189.044322 124.087049) (width 0.2) (layer "F.Cu") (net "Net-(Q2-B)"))
 (segment (start 103.044322 82.587049) (end 103.044322 95.587049) (width 0.2) (layer "F.Cu") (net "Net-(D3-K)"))
 (segment (start 94.044322 82.587049) (end 103.044322 82.587049) (width 0.2) (layer "F.Cu") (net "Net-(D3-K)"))
 (segment (start 103.044322 95.587049) (end 99.354322 95.587049) (width 0.2) (layer "F.Cu") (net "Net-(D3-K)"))
 (segment (start 94.044322 77.587049) (end 94.044322 82.587049) (width 0.2) (layer "F.Cu") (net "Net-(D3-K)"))
 (segment (start 82.094322 77.537049) (end 93.994322 77.537049) (width 0.2) (layer "F.Cu") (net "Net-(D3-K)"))
 (segment (start 93.994322 77.537049) (end 94.044322 77.587049) (width 0.2) (layer "F.Cu") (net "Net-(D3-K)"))
 (segment (start 182.454322 121.587049) (end 182.314322 121.447049) (width 0.2) (layer "F.Cu") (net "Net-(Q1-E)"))
 (segment (start 178.044322 128.587049) (end 125.544322 128.587049) (width 0.2) (layer "F.Cu") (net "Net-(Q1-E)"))
 (segment (start 182.454322 121.587049) (end 182.544322 121.587049) (width 0.2) (layer "F.Cu") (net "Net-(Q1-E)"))
 (segment (start 125.544322 128.587049) (end 125.544322 126.341414) (width 0.2) (layer "F.Cu") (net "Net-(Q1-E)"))
 (segment (start 125.544322 126.341414) (end 130.438687 121.447049) (width 0.2) (layer "F.Cu") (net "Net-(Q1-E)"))
 (segment (start 178.544322 120.802049) (end 178.544322 128.087049) (width 0.2) (layer "F.Cu") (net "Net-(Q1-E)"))
 (segment (start 182.314322 121.447049) (end 182.314322 121.325323) (width 0.2) (layer "F.Cu") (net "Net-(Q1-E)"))
 (segment (start 178.544322 128.087049) (end 178.044322 128.587049) (width 0.2) (layer "F.Cu") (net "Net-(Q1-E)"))
 (segment (start 130.438687 121.447049) (end 135.774322 121.447049) (width 0.2) (layer "F.Cu") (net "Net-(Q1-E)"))
 (segment (start 182.314322 121.325323) (end 181.386048 120.397049) (width 0.2) (layer "F.Cu") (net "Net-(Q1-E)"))
 (segment (start 181.386048 120.397049) (end 178.949322 120.397049) (width 0.2) (layer "F.Cu") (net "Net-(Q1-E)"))
 (segment (start 178.949322 120.397049) (end 178.544322 120.802049) (width 0.2) (layer "F.Cu") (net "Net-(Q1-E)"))
 (segment (start 129.544322 116.277049) (end 132.824322 116.277049) (width 0.2) (layer "F.Cu") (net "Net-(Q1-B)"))
 (segment (start 132.824322 116.277049) (end 137.044322 120.497049) (width 0.2) (layer "F.Cu") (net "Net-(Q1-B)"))
 (segment (start 137.044322 120.497049) (end 137.044322 121.447049) (width 0.2) (layer "F.Cu") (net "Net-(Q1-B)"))
 (segment (start 143.234322 123.897049) (end 143.794322 123.337049) (width 0.2) (layer "F.Cu") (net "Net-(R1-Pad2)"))
 (segment (start 150.294322 123.337049) (end 143.794322 123.337049) (width 0.2) (layer "F.Cu") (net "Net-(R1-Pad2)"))
 (segment (start 150.544322 123.587049) (end 150.294322 123.337049) (width 0.2) (layer "F.Cu") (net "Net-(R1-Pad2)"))
 (segment (start 129.544322 123.897049) (end 143.234322 123.897049) (width 0.2) (layer "F.Cu") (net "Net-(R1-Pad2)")))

